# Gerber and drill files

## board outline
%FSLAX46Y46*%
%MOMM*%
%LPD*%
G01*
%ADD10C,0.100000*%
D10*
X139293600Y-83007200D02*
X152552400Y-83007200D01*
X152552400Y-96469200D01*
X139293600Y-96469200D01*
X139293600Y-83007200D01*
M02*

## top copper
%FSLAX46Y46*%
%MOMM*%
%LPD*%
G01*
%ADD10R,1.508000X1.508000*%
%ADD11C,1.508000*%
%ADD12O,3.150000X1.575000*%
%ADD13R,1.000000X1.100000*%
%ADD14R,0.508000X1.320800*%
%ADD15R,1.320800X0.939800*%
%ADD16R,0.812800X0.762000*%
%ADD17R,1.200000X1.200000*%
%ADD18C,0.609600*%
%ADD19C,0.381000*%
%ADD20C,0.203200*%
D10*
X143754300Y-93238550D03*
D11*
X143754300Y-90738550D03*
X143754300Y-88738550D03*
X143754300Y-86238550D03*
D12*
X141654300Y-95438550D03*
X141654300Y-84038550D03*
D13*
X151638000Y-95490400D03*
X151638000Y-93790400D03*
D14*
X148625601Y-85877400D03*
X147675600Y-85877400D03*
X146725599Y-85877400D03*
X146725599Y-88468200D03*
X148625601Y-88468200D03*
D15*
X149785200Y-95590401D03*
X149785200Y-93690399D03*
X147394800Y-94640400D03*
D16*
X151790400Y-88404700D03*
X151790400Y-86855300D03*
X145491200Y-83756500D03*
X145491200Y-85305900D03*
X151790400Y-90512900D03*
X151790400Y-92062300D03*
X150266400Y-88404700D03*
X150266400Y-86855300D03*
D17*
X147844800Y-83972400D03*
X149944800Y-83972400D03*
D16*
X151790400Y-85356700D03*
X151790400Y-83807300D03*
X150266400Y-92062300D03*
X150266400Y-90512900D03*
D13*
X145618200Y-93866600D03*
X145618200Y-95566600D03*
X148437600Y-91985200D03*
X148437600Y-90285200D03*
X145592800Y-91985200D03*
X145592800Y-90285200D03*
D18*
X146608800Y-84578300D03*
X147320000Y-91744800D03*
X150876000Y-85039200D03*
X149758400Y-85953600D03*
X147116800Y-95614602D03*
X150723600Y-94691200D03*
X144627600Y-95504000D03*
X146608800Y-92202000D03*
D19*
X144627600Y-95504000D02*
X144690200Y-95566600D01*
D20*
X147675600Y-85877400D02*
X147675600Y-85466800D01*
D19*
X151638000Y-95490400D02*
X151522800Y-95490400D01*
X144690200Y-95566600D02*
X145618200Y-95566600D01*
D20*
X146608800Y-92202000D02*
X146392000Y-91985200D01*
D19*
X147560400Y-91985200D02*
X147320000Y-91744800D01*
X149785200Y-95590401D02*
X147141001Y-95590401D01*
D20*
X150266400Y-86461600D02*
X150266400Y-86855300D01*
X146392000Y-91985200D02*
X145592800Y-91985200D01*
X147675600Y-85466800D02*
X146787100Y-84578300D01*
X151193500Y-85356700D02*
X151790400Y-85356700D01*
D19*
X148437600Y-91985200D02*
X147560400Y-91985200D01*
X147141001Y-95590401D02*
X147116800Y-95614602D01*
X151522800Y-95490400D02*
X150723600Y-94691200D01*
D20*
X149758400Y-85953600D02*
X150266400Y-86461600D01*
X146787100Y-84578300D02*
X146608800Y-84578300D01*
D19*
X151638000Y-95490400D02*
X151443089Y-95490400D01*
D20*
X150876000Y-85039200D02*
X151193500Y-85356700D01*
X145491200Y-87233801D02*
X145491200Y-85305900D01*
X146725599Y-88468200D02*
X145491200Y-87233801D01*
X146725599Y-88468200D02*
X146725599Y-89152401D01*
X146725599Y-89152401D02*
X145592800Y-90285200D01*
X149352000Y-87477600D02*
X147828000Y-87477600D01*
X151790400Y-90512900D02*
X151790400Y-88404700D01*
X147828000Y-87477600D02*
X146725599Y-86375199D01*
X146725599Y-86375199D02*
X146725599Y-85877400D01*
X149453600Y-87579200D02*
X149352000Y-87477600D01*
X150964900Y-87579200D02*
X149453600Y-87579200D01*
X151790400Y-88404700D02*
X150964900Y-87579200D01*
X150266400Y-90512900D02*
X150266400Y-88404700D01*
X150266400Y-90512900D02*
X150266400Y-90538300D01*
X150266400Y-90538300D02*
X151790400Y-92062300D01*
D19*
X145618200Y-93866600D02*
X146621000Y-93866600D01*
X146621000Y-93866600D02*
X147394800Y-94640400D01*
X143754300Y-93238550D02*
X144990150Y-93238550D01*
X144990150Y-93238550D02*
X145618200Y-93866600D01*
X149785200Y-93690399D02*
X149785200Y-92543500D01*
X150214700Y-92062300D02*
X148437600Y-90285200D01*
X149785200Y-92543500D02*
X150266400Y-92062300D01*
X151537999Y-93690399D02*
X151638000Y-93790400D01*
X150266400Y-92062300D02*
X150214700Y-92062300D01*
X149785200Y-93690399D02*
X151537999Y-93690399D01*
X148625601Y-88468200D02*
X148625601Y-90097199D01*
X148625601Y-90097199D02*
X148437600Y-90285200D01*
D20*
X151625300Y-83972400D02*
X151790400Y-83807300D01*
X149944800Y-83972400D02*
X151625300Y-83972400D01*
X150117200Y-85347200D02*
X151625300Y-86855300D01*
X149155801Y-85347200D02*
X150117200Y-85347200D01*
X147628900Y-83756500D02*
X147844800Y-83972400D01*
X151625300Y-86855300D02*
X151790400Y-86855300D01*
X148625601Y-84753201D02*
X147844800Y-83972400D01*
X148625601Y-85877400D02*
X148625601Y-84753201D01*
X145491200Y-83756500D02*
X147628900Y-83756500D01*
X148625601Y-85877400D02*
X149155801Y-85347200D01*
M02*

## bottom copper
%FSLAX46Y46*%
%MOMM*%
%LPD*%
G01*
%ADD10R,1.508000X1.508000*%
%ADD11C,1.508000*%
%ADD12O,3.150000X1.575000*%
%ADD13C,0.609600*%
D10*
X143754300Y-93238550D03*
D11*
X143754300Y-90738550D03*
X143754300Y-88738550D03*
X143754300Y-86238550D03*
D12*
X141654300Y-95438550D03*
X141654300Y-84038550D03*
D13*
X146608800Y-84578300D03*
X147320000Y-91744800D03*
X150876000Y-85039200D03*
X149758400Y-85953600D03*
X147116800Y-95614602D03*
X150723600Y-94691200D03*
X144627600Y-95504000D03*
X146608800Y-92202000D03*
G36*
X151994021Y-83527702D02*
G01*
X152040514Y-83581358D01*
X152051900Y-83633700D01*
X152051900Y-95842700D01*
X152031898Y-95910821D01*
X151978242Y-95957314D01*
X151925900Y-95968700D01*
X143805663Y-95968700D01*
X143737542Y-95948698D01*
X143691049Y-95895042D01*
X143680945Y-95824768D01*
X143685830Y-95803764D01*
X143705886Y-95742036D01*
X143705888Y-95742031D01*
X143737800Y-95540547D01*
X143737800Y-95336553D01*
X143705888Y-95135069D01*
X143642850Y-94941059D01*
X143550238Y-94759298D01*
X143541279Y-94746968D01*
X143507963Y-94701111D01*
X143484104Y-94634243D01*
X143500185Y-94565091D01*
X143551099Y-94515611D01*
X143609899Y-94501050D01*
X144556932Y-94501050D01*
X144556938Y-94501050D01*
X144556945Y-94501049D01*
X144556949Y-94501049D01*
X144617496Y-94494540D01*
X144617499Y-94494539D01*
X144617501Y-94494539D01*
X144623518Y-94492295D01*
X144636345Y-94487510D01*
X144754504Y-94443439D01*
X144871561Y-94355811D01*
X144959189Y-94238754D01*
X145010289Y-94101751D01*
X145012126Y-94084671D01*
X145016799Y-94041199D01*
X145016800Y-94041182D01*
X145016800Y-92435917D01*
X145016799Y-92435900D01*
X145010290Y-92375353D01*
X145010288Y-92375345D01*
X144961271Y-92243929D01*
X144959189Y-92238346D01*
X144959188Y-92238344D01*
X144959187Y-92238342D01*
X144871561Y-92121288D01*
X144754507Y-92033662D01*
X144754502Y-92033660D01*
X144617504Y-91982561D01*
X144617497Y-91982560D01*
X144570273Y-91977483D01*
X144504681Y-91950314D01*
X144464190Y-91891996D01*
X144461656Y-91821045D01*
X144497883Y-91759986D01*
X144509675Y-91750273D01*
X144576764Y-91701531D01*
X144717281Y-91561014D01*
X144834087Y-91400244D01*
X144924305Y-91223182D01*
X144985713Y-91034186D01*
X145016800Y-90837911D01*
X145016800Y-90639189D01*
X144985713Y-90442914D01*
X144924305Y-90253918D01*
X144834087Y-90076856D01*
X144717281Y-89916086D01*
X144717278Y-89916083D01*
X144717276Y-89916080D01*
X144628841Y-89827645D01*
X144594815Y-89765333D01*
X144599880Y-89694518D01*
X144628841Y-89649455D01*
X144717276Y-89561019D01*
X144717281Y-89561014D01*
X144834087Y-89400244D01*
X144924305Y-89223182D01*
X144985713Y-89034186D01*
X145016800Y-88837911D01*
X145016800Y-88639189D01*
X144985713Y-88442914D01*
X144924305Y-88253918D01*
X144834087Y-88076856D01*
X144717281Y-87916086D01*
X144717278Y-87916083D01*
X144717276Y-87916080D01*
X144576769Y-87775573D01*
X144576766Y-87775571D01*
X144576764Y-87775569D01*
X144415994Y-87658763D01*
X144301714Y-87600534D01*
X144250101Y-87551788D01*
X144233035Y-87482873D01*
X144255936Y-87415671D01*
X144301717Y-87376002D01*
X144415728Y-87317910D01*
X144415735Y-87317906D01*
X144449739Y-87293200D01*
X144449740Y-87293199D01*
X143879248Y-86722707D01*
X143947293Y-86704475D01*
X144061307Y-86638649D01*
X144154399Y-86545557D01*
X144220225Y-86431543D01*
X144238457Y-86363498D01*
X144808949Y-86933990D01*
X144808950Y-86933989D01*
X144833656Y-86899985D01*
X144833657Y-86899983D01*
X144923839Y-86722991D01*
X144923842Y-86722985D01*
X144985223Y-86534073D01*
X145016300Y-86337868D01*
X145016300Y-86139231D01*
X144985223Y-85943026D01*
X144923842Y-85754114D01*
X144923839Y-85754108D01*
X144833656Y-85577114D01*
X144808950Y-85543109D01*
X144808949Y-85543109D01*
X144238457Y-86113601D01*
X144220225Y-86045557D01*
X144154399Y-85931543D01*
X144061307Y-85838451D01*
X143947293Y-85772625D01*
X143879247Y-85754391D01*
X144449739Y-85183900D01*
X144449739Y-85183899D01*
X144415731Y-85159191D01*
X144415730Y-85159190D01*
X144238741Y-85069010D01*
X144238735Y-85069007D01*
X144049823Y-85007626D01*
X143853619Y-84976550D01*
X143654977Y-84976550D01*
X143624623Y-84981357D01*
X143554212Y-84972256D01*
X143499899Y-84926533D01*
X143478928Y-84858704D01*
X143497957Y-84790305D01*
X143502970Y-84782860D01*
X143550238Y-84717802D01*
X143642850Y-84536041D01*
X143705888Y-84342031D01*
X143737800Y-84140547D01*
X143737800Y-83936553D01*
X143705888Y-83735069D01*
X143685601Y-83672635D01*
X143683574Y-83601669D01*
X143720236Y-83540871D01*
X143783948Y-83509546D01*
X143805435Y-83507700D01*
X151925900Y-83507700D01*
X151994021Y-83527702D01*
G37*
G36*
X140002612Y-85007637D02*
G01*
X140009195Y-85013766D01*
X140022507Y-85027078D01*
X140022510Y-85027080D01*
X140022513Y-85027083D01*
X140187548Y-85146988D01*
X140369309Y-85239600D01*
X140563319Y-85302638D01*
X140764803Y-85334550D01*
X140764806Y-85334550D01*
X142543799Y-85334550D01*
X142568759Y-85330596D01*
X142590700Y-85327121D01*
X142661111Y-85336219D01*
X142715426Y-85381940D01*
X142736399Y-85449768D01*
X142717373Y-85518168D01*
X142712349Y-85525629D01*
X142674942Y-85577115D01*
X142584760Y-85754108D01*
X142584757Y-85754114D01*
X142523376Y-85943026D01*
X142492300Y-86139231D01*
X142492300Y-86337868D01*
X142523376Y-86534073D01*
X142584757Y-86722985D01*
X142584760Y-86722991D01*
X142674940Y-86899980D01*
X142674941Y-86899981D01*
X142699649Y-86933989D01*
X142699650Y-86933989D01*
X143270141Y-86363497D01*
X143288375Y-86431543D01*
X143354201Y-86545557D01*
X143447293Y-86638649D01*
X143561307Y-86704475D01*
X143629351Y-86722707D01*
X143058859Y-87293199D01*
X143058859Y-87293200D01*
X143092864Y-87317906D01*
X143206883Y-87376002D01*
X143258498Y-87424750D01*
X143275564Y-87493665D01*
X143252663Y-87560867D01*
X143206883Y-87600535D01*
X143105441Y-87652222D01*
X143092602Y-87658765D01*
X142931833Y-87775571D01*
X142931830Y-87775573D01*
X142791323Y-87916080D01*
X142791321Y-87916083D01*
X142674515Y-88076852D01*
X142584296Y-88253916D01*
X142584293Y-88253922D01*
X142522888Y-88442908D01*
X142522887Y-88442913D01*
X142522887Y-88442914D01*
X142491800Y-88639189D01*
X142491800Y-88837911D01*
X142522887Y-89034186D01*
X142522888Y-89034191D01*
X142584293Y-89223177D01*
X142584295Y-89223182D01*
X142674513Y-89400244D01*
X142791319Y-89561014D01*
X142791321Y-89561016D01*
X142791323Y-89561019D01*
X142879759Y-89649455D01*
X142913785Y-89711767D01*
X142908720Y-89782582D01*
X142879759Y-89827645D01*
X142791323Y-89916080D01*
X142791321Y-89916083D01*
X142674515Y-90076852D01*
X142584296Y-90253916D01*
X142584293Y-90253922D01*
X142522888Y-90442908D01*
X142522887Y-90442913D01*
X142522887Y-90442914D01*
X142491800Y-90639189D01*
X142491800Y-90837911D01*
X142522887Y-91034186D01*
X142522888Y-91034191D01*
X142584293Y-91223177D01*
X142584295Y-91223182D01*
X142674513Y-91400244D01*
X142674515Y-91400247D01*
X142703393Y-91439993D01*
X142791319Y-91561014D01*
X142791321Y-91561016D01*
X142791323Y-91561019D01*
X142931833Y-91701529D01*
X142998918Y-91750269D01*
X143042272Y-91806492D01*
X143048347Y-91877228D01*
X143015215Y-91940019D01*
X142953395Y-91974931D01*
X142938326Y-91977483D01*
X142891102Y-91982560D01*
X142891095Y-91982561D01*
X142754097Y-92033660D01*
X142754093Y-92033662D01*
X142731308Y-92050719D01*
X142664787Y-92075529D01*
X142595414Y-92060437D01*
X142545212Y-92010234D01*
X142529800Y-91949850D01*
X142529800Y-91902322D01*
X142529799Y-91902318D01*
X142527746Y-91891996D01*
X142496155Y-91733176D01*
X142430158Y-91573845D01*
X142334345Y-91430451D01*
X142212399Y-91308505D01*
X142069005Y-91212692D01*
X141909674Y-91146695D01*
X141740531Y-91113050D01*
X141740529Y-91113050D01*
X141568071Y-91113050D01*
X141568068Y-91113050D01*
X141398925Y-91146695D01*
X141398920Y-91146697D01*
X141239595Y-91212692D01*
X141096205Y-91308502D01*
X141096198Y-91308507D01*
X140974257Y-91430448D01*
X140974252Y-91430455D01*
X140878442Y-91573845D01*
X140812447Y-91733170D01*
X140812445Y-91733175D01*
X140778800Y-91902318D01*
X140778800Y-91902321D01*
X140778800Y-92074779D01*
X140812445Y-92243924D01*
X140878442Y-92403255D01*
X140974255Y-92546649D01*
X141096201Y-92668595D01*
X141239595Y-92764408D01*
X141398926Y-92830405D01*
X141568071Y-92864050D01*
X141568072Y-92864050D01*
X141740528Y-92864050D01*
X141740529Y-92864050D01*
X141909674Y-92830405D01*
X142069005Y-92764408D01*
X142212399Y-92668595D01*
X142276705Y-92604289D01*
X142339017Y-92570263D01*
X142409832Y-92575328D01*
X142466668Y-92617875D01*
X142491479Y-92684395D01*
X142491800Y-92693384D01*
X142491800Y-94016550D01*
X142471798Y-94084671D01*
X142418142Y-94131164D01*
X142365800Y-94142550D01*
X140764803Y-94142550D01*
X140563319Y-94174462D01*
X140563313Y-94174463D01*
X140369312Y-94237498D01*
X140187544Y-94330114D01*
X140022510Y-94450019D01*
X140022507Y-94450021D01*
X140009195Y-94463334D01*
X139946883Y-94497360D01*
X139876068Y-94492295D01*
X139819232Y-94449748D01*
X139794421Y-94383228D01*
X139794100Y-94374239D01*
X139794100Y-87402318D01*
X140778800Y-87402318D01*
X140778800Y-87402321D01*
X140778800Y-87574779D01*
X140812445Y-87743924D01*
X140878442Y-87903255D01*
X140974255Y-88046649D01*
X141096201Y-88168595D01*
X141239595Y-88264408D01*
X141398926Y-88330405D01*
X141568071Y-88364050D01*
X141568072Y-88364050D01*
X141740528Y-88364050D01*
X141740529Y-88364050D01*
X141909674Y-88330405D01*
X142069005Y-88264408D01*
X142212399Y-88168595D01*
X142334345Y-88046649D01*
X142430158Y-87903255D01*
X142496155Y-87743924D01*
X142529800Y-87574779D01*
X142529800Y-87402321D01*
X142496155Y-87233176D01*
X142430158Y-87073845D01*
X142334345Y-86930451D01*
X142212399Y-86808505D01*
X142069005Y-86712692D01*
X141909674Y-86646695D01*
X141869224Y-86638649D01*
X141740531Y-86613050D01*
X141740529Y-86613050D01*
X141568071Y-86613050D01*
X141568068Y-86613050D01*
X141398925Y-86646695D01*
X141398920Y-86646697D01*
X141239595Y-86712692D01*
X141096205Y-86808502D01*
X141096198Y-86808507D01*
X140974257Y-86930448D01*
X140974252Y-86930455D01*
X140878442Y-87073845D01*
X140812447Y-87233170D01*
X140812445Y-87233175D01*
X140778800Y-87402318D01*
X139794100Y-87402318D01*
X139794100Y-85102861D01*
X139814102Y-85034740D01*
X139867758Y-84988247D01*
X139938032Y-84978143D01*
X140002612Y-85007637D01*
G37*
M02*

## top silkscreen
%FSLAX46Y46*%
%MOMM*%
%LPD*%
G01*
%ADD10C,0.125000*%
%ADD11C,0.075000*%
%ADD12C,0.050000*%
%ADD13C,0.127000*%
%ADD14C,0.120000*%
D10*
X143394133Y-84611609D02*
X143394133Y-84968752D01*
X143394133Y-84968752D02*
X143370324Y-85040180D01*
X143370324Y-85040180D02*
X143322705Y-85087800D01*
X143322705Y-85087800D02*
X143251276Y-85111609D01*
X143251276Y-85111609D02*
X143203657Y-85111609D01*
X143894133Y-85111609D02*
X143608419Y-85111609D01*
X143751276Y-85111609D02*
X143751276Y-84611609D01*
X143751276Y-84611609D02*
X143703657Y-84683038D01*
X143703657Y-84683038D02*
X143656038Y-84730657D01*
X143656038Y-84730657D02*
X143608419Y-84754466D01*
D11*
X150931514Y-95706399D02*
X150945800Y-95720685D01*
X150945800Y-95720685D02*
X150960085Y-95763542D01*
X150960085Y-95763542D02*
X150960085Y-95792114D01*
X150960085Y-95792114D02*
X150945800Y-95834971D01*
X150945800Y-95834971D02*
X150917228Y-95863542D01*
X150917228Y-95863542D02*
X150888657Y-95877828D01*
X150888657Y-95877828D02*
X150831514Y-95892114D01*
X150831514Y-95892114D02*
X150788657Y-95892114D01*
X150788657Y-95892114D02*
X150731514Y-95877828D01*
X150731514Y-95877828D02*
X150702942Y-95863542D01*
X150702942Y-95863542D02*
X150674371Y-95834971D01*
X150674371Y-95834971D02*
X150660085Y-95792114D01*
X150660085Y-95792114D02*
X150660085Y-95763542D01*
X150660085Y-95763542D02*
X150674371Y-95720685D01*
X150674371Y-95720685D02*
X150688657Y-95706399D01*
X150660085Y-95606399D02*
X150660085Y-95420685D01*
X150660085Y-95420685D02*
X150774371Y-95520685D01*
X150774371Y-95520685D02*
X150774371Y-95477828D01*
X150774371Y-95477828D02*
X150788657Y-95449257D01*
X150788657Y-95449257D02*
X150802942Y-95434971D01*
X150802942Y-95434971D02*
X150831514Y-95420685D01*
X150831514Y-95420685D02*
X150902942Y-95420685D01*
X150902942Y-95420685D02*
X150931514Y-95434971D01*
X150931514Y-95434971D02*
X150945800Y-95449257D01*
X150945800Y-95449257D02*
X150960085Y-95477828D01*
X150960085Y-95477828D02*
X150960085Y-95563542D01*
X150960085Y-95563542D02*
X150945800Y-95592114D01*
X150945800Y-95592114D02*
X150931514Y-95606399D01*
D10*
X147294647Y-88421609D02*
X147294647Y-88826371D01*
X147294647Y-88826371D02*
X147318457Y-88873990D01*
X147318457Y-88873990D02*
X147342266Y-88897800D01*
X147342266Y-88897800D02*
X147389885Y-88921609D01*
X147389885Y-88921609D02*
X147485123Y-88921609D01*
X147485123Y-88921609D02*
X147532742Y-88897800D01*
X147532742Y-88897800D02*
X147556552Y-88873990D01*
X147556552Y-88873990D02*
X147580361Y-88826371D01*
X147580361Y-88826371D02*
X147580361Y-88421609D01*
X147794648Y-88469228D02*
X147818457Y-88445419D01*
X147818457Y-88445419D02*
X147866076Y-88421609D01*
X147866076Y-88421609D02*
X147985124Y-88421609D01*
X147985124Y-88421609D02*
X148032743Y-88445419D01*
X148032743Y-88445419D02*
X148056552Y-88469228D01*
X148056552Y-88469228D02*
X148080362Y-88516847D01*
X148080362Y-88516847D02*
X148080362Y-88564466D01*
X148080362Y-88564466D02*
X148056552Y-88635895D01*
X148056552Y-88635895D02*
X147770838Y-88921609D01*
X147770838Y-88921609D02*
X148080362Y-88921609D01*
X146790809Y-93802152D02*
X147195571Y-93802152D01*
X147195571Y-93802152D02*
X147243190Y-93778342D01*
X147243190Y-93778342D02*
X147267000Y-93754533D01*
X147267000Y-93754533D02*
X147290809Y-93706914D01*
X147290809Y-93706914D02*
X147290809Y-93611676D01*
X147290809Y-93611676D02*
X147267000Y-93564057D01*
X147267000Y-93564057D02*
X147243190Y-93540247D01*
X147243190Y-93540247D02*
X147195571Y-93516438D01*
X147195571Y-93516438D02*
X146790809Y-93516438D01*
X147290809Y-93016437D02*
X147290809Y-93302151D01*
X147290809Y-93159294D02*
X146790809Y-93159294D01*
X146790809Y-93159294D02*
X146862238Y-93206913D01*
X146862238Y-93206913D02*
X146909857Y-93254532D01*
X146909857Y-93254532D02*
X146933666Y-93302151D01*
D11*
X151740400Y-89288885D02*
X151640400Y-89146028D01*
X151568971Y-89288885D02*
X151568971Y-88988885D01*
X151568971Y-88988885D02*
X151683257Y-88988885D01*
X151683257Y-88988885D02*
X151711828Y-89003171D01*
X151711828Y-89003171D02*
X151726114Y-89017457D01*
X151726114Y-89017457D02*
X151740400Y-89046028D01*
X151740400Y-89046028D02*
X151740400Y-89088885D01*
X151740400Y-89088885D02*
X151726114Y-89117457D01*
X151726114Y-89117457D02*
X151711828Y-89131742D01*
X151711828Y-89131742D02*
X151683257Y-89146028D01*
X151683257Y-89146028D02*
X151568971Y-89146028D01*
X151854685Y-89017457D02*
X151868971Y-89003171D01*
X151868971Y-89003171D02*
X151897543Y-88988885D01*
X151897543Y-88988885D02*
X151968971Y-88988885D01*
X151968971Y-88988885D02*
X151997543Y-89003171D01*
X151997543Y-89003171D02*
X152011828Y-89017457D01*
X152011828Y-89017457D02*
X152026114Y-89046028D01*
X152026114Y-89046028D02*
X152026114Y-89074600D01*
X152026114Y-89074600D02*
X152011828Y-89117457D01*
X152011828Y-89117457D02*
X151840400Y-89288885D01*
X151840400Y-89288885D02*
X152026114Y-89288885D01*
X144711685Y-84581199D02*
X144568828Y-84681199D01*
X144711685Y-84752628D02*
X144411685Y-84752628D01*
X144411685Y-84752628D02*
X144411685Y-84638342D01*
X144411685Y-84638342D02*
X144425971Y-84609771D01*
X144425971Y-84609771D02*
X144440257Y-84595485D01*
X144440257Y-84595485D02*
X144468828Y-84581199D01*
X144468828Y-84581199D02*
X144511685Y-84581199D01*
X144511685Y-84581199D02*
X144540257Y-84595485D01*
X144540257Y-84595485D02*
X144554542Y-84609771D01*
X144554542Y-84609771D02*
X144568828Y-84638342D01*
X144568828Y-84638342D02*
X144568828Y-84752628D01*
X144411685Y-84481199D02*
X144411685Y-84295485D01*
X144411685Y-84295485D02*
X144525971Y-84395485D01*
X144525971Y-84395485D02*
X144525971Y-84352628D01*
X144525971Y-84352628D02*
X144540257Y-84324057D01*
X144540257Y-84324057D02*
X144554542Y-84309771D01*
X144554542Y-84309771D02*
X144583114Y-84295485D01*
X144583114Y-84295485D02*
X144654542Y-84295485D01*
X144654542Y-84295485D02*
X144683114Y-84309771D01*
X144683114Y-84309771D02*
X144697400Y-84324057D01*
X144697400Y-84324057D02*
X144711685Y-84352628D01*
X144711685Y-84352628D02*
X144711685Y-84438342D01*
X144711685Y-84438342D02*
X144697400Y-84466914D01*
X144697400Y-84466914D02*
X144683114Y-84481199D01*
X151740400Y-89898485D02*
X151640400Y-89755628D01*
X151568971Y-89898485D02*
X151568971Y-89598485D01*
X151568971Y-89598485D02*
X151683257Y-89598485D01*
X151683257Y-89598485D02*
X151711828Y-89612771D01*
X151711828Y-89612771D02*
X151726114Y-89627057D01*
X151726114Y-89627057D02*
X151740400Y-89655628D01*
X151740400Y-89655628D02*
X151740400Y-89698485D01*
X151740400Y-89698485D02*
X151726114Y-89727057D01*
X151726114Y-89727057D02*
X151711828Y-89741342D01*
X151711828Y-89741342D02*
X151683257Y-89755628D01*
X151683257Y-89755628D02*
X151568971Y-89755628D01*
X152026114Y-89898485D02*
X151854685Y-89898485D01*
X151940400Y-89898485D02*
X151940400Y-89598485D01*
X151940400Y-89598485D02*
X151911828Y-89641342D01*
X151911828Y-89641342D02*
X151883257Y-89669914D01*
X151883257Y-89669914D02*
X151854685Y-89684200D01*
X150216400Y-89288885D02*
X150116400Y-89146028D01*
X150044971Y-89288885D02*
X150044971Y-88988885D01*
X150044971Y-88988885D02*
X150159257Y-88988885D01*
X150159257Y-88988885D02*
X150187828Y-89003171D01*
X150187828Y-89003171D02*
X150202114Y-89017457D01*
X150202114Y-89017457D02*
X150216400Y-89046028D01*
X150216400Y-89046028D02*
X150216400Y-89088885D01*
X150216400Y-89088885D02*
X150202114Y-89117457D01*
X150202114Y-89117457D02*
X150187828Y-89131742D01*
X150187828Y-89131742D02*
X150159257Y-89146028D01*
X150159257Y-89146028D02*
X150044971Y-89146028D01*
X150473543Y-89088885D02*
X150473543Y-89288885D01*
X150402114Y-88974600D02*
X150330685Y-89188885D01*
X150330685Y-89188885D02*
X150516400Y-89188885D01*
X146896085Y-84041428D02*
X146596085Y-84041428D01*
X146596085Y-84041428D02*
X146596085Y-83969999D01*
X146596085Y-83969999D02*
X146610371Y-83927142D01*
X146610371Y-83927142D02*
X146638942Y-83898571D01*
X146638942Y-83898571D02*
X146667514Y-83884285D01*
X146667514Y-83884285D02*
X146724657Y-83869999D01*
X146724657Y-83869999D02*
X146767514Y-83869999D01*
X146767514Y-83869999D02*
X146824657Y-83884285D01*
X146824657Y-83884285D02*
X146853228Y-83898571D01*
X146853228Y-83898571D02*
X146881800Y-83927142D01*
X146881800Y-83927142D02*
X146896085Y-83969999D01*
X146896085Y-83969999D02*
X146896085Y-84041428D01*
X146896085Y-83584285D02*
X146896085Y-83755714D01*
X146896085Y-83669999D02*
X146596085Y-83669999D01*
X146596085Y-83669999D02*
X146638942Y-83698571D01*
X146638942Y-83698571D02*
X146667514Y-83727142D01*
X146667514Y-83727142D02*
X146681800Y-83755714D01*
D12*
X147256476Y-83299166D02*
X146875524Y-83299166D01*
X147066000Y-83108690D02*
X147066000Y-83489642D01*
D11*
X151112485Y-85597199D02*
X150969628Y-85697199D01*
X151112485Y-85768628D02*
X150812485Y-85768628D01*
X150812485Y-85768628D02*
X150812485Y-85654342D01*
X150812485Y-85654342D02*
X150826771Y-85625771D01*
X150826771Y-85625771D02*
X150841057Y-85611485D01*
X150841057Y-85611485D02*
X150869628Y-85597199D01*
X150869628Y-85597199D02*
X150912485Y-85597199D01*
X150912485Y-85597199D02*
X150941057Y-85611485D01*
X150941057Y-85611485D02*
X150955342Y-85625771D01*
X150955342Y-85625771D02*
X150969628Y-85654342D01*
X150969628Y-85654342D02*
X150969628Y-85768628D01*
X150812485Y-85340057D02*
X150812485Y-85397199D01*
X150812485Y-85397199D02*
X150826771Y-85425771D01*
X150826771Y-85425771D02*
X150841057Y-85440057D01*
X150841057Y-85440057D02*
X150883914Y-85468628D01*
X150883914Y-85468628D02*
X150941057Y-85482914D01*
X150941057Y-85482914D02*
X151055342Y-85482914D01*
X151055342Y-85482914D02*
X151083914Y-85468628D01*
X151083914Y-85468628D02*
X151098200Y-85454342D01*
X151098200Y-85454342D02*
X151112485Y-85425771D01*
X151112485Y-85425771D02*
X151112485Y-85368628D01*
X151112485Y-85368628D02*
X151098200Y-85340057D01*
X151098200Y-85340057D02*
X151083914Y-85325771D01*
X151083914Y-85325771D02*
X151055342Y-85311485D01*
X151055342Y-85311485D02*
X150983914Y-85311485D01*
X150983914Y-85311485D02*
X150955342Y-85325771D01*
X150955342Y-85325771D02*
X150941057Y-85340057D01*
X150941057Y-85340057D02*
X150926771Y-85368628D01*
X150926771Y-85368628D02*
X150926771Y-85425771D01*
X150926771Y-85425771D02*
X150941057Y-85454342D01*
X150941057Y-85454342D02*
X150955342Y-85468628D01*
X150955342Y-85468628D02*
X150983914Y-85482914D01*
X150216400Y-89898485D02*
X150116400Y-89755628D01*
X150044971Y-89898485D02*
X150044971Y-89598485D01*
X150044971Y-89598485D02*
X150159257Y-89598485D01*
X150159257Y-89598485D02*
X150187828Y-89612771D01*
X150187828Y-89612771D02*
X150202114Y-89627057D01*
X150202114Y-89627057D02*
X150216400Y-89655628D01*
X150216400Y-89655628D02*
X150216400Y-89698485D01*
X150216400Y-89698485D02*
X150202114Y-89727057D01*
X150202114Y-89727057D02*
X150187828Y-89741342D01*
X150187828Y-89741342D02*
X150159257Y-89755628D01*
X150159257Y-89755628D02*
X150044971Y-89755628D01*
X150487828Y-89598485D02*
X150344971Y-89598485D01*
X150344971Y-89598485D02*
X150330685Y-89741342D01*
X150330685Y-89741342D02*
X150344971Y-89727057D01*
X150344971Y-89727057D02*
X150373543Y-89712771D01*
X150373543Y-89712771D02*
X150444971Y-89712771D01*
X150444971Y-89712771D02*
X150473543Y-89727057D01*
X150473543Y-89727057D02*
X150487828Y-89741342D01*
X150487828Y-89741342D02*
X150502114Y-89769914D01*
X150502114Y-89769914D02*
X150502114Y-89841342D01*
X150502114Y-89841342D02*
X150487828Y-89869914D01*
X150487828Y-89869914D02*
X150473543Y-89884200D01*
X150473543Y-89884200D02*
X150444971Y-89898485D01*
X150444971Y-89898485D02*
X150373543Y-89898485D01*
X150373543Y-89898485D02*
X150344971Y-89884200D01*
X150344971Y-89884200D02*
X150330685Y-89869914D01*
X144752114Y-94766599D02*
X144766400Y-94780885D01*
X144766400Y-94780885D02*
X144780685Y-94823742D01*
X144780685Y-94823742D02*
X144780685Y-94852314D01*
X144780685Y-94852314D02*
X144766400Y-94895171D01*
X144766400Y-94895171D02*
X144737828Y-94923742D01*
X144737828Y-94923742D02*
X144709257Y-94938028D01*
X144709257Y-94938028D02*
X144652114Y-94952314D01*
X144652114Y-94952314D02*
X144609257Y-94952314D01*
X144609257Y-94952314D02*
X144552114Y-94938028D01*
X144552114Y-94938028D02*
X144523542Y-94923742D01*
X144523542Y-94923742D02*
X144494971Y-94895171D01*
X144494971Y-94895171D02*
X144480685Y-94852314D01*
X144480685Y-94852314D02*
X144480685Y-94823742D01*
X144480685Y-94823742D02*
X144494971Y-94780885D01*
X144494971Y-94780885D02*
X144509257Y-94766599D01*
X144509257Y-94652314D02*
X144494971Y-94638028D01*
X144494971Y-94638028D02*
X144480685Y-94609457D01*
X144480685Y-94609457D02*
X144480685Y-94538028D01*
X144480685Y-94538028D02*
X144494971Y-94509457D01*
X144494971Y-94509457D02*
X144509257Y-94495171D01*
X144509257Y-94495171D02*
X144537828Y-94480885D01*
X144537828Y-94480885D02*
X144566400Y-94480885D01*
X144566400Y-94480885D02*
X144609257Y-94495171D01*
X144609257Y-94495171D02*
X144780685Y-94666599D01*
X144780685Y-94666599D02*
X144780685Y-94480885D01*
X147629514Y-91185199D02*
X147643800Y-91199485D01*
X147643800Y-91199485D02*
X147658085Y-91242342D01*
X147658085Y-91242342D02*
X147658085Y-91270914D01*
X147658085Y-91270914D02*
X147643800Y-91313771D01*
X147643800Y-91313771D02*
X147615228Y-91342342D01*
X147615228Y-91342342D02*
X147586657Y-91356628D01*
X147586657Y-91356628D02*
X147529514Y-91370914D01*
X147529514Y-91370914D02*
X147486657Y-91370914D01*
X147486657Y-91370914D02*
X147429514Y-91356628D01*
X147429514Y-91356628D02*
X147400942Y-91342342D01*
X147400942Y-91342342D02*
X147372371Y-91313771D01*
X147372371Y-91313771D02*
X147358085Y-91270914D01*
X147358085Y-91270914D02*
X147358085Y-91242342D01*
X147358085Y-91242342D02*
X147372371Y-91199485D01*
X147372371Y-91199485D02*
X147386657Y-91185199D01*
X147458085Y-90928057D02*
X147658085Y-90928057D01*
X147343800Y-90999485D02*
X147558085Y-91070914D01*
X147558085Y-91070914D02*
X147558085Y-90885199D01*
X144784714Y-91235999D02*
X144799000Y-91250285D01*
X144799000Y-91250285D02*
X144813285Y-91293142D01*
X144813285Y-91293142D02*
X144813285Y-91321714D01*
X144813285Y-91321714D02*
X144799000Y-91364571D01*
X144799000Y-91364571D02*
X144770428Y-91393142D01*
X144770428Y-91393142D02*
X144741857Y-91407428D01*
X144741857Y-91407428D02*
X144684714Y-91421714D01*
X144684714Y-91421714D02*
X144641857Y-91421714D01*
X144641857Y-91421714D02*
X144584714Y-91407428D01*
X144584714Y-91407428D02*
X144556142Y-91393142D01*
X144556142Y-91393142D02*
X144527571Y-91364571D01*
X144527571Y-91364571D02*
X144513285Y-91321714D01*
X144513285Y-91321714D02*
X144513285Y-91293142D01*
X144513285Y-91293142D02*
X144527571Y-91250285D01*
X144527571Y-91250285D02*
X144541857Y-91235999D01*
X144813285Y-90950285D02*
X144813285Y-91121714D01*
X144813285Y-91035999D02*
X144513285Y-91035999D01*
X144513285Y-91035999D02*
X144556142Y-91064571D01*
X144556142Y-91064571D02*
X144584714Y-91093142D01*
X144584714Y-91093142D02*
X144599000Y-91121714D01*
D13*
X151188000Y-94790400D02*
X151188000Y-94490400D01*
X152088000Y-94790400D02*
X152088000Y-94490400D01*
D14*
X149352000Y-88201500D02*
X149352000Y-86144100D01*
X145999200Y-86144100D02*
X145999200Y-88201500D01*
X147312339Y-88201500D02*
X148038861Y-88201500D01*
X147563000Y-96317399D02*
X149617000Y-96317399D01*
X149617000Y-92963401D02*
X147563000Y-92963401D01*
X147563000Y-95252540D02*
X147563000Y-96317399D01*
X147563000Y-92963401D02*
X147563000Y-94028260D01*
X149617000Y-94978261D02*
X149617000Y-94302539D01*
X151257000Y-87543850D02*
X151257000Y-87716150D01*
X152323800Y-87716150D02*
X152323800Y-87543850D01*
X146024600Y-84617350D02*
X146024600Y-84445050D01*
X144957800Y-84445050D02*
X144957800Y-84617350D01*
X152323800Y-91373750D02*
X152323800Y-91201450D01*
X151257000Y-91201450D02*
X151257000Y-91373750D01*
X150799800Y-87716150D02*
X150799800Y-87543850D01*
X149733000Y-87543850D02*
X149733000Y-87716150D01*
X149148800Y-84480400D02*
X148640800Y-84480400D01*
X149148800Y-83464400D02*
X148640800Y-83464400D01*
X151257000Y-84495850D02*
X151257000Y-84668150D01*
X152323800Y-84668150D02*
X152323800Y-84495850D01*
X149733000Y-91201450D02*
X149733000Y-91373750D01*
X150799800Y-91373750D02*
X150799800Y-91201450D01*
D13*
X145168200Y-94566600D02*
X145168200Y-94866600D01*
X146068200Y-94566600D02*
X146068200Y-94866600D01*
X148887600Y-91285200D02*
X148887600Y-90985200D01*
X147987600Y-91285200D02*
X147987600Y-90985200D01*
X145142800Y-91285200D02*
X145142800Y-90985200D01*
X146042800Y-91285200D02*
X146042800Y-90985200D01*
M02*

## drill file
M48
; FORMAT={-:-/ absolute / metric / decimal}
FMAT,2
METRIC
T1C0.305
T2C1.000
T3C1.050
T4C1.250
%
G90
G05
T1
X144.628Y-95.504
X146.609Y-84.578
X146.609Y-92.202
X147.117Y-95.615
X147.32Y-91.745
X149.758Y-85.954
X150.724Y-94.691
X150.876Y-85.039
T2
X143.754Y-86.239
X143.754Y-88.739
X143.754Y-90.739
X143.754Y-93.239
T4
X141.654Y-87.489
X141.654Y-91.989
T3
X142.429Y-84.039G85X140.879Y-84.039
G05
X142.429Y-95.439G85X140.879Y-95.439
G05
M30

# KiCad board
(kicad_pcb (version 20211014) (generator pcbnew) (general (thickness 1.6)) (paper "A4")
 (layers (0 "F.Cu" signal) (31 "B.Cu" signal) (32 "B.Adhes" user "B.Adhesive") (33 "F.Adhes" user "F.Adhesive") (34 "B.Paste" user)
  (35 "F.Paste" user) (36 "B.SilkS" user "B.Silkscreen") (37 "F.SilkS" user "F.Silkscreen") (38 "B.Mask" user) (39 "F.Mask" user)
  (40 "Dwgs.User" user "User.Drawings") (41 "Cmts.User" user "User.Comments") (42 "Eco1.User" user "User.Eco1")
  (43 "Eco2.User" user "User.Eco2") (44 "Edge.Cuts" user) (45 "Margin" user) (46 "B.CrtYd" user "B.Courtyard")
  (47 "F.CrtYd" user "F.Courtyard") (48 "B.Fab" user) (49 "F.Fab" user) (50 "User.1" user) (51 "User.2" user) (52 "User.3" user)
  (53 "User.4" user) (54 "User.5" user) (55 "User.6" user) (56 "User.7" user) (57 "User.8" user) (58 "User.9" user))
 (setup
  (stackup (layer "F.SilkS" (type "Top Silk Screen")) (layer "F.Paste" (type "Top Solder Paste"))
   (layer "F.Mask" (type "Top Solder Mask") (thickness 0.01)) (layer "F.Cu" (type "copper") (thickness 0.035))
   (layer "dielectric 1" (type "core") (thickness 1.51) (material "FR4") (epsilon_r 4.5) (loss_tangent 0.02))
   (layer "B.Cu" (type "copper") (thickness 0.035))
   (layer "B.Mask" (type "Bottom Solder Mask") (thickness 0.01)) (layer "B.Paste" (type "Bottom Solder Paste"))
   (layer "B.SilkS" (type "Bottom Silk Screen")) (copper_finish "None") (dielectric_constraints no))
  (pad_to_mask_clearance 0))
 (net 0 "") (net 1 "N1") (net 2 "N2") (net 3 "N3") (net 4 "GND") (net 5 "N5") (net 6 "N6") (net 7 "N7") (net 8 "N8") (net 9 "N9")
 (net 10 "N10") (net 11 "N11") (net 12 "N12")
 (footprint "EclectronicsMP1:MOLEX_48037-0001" (layer "F.Cu") (at 141.6543 89.73855 -90)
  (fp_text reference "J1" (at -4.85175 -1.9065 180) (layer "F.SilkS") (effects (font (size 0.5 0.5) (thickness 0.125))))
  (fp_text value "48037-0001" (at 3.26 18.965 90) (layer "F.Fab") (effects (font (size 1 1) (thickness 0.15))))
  (pad "" np_thru_hole circle (at -2.25 0 270) (size 1.25 1.25) (drill 1.25) (layers *.Cu *.Mask))
  (pad "" np_thru_hole circle (at 2.25 0 270) (size 1.25 1.25) (drill 1.25) (layers *.Cu *.Mask))
  (pad "1" thru_hole rect (at 3.5 -2.1 270) (size 1.508 1.508) (drill 1) (layers *.Cu *.Mask) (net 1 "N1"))
  (pad "2" thru_hole circle (at 1 -2.1 270) (size 1.508 1.508) (drill 1) (layers *.Cu *.Mask) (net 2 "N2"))
  (pad "3" thru_hole circle (at -1 -2.1 270) (size 1.508 1.508) (drill 1) (layers *.Cu *.Mask) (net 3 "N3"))
  (pad "4" thru_hole circle (at -3.5 -2.1 270) (size 1.508 1.508) (drill 1) (layers *.Cu *.Mask) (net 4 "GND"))
  (pad "S1" thru_hole oval (at 5.7 0 270) (size 1.575 3.15) (drill oval 1.05 2.6) (layers *.Cu *.Mask) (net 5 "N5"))
  (pad "S2" thru_hole oval (at -5.7 0 270) (size 1.575 3.15) (drill oval 1.05 2.6) (layers *.Cu *.Mask) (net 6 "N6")))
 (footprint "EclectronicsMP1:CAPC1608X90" (layer "F.Cu") (at 151.638 94.6404 90)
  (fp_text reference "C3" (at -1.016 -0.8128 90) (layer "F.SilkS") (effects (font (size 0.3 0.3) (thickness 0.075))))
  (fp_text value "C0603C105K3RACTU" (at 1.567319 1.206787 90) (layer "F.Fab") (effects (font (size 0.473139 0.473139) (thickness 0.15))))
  (fp_line (start -0.15 -0.45) (end 0.15 -0.45) (layer "F.SilkS") (width 0.127))
  (fp_line (start -0.15 0.45) (end 0.15 0.45) (layer "F.SilkS") (width 0.127))
  (pad "1" smd rect (at -0.85 0 90) (size 1.1 1) (layers "F.Cu" "F.Paste" "F.Mask") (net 4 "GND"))
  (pad "2" smd rect (at 0.85 0 90) (size 1.1 1) (layers "F.Cu" "F.Paste" "F.Mask") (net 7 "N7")))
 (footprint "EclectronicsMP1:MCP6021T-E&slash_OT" (layer "F.Cu") (at 147.6756 87.1728 -90)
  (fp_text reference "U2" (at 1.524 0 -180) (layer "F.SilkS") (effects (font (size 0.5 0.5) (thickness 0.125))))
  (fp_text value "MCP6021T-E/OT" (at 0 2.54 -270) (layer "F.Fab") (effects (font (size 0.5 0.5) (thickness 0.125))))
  (fp_line (start 1.0287 -1.6764) (end -1.0287 -1.6764) (layer "F.SilkS") (width 0.12))
  (fp_line (start -1.0287 1.6764) (end 1.0287 1.6764) (layer "F.SilkS") (width 0.12))
  (fp_line (start 1.0287 0.363261) (end 1.0287 -0.363261) (layer "F.SilkS") (width 0.12))
  (pad "1" smd rect (at -1.2954 -0.950001 270) (size 1.3208 0.508) (layers "F.Cu" "F.Paste" "F.Mask") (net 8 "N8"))
  (pad "2" smd rect (at -1.2954 0 270) (size 1.3208 0.508) (layers "F.Cu" "F.Paste" "F.Mask") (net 4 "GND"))
  (pad "3" smd rect (at -1.2954 0.950001 270) (size 1.3208 0.508) (layers "F.Cu" "F.Paste" "F.Mask") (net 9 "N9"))
  (pad "4" smd rect (at 1.2954 0.950001 270) (size 1.3208 0.508) (layers "F.Cu" "F.Paste" "F.Mask") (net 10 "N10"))
  (pad "5" smd rect (at 1.2954 -0.950001 270) (size 1.3208 0.508) (layers "F.Cu" "F.Paste" "F.Mask") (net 7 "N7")))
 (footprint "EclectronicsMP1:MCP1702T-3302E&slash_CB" (layer "F.Cu") (at 148.59 94.6404 90)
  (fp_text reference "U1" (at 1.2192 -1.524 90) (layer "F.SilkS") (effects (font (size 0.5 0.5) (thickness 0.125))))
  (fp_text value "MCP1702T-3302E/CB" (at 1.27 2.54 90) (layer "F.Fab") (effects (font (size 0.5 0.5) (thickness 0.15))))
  (fp_line (start -1.676999 -1.027) (end -1.676999 1.027) (layer "F.SilkS") (width 0.12))
  (fp_line (start 1.676999 1.027) (end 1.676999 -1.027) (layer "F.SilkS") (width 0.12))
  (fp_line (start -0.61214 -1.027) (end -1.676999 -1.027) (layer "F.SilkS") (width 0.12))
  (fp_line (start 1.676999 -1.027) (end 0.61214 -1.027) (layer "F.SilkS") (width 0.12))
  (fp_line (start -0.337861 1.027) (end 0.337861 1.027) (layer "F.SilkS") (width 0.12))
  (pad "1" smd rect (at -0.950001 1.1952 90) (size 0.9398 1.3208) (layers "F.Cu" "F.Paste" "F.Mask") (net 4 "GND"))
  (pad "2" smd rect (at 0.950001 1.1952 90) (size 0.9398 1.3208) (layers "F.Cu" "F.Paste" "F.Mask") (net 7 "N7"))
  (pad "3" smd rect (at 0 -1.1952 90) (size 0.9398 1.3208) (layers "F.Cu" "F.Paste" "F.Mask") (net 1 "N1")))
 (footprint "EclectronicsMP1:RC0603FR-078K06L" (layer "F.Cu") (at 151.7904 87.63 90)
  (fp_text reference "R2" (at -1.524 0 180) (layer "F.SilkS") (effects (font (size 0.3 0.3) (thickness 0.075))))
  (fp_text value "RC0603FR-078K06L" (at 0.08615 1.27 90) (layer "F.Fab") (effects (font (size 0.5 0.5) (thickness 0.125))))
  (fp_line (start 0.08615 -0.5334) (end -0.08615 -0.5334) (layer "F.SilkS") (width 0.12))
  (fp_line (start -0.08615 0.5334) (end 0.08615 0.5334) (layer "F.SilkS") (width 0.12))
  (pad "1" smd rect (at -0.7747 0 90) (size 0.762 0.8128) (layers "F.Cu" "F.Paste" "F.Mask") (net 9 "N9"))
  (pad "2" smd rect (at 0.7747 0 90) (size 0.762 0.8128) (layers "F.Cu" "F.Paste" "F.Mask") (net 8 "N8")))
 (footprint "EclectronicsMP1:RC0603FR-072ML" (layer "F.Cu") (at 145.4912 84.5312 -90)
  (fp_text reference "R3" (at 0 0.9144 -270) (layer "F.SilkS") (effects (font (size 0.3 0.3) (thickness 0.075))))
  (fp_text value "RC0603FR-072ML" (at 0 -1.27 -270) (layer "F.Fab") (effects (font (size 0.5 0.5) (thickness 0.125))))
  (fp_line (start 0.08615 -0.5334) (end -0.08615 -0.5334) (layer "F.SilkS") (width 0.12))
  (fp_line (start -0.08615 0.5334) (end 0.08615 0.5334) (layer "F.SilkS") (width 0.12))
  (pad "1" smd rect (at -0.7747 0 270) (size 0.762 0.8128) (layers "F.Cu" "F.Paste" "F.Mask") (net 8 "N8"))
  (pad "2" smd rect (at 0.7747 0 270) (size 0.762 0.8128) (layers "F.Cu" "F.Paste" "F.Mask") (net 10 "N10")))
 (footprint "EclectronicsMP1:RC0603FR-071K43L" (layer "F.Cu") (at 151.7904 91.2876 -90)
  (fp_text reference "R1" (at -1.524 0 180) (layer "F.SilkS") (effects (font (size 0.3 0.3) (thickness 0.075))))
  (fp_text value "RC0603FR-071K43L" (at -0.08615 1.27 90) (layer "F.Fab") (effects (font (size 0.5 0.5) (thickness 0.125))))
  (fp_line (start 0.08615 -0.5334) (end -0.08615 -0.5334) (layer "F.SilkS") (width 0.12))
  (fp_line (start -0.08615 0.5334) (end 0.08615 0.5334) (layer "F.SilkS") (width 0.12))
  (pad "1" smd rect (at -0.7747 0 270) (size 0.762 0.8128) (layers "F.Cu" "F.Paste" "F.Mask") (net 9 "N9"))
  (pad "2" smd rect (at 0.7747 0 270) (size 0.762 0.8128) (layers "F.Cu" "F.Paste" "F.Mask") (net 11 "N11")))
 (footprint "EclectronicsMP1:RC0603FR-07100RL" (layer "F.Cu") (at 150.2664 87.63 90)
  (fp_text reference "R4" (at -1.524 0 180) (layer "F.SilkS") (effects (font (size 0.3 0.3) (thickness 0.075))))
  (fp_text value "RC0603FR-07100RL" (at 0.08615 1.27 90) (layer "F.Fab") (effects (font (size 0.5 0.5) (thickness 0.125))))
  (fp_line (start -0.08615 0.5334) (end 0.08615 0.5334) (layer "F.SilkS") (width 0.12))
  (fp_line (start 0.08615 -0.5334) (end -0.08615 -0.5334) (layer "F.SilkS") (width 0.12))
  (pad "1" smd rect (at -0.7747 0 90) (size 0.762 0.8128) (layers "F.Cu" "F.Paste" "F.Mask") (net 11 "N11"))
  (pad "2" smd rect (at 0.7747 0 90) (size 0.762 0.8128) (layers "F.Cu" "F.Paste" "F.Mask") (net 4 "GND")))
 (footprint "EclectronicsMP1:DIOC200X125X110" (layer "F.Cu") (at 148.8948 83.9724 180)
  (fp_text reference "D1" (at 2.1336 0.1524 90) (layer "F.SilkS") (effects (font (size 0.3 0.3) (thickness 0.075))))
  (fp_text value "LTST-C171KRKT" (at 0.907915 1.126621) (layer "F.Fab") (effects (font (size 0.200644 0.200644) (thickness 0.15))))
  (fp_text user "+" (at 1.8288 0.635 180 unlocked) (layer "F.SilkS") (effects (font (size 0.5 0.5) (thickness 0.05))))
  (fp_line (start -0.254 -0.508) (end 0.254 -0.508) (layer "F.SilkS") (width 0.12))
  (fp_line (start -0.254 0.508) (end 0.254 0.508) (layer "F.SilkS") (width 0.12))
  (pad "+" smd rect (at 1.05 0 180) (size 1.2 1.2) (layers "F.Cu" "F.Paste" "F.Mask") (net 8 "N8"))
  (pad "-" smd rect (at -1.05 0 180) (size 1.2 1.2) (layers "F.Cu" "F.Paste" "F.Mask") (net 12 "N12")))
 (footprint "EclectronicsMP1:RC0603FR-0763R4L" (layer "F.Cu") (at 151.7904 84.582 90)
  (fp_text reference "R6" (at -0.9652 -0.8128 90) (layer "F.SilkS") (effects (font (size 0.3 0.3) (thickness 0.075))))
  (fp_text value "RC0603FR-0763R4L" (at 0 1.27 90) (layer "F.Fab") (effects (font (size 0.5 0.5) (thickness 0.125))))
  (fp_line (start 0.08615 -0.5334) (end -0.08615 -0.5334) (layer "F.SilkS") (width 0.12))
  (fp_line (start -0.08615 0.5334) (end 0.08615 0.5334) (layer "F.SilkS") (width 0.12))
  (pad "1" smd rect (at -0.7747 0 90) (size 0.762 0.8128) (layers "F.Cu" "F.Paste" "F.Mask") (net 4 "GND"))
  (pad "2" smd rect (at 0.7747 0 90) (size 0.762 0.8128) (layers "F.Cu" "F.Paste" "F.Mask") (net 12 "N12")))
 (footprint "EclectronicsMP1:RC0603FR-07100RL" (layer "F.Cu") (at 150.2664 91.2876 90)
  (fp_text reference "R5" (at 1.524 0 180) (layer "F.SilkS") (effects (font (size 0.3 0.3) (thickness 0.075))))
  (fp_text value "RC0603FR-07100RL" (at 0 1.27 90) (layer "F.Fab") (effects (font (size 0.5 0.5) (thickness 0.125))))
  (fp_line (start 0.08615 -0.5334) (end -0.08615 -0.5334) (layer "F.SilkS") (width 0.12))
  (fp_line (start -0.08615 0.5334) (end 0.08615 0.5334) (layer "F.SilkS") (width 0.12))
  (pad "1" smd rect (at -0.7747 0 90) (size 0.762 0.8128) (layers "F.Cu" "F.Paste" "F.Mask") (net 7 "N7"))
  (pad "2" smd rect (at 0.7747 0 90) (size 0.762 0.8128) (layers "F.Cu" "F.Paste" "F.Mask") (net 11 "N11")))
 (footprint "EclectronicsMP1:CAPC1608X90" (layer "F.Cu") (at 145.6182 94.7166 -90)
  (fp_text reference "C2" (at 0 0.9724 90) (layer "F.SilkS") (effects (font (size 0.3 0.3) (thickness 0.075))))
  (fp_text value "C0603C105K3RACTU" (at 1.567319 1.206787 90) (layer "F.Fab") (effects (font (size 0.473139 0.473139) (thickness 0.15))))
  (fp_line (start -0.15 0.45) (end 0.15 0.45) (layer "F.SilkS") (width 0.127))
  (fp_line (start -0.15 -0.45) (end 0.15 -0.45) (layer "F.SilkS") (width 0.127))
  (pad "1" smd rect (at -0.85 0 270) (size 1.1 1) (layers "F.Cu" "F.Paste" "F.Mask") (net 1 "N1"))
  (pad "2" smd rect (at 0.85 0 270) (size 1.1 1) (layers "F.Cu" "F.Paste" "F.Mask") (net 4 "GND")))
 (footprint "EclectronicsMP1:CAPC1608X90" (layer "F.Cu") (at 148.4376 91.1352 90)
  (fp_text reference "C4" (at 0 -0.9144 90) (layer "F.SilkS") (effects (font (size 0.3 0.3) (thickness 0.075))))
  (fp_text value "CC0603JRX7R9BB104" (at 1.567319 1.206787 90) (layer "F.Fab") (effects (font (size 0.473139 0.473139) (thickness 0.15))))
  (fp_line (start -0.15 0.45) (end 0.15 0.45) (layer "F.SilkS") (width 0.127))
  (fp_line (start -0.15 -0.45) (end 0.15 -0.45) (layer "F.SilkS") (width 0.127))
  (pad "1" smd rect (at -0.85 0 90) (size 1.1 1) (layers "F.Cu" "F.Paste" "F.Mask") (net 4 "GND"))
  (pad "2" smd rect (at 0.85 0 90) (size 1.1 1) (layers "F.Cu" "F.Paste" "F.Mask") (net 7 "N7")))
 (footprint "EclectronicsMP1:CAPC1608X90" (layer "F.Cu") (at 145.5928 91.1352 90)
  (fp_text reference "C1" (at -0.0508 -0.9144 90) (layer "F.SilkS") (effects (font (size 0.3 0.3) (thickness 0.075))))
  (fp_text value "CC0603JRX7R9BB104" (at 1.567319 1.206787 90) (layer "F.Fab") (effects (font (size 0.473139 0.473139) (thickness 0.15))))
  (fp_line (start -0.15 -0.45) (end 0.15 -0.45) (layer "F.SilkS") (width 0.127))
  (fp_line (start -0.15 0.45) (end 0.15 0.45) (layer "F.SilkS") (width 0.127))
  (pad "1" smd rect (at -0.85 0 90) (size 1.1 1) (layers "F.Cu" "F.Paste" "F.Mask") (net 4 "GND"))
  (pad "2" smd rect (at 0.85 0 90) (size 1.1 1) (layers "F.Cu" "F.Paste" "F.Mask") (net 10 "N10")))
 (gr_rect (start 152.5524 96.4692) (end 139.2936 83.0072) (layer "Edge.Cuts") (width 0.1) (fill none))
 (segment (start 144.6276 95.504) (end 144.6902 95.5666) (width 0.381) (layer "F.Cu") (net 4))
 (segment (start 147.6756 85.8774) (end 147.6756 85.4668) (width 0.2032) (layer "F.Cu") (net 4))
 (segment (start 151.638 95.4904) (end 151.5228 95.4904) (width 0.381) (layer "F.Cu") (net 4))
 (segment (start 144.6902 95.5666) (end 145.6182 95.5666) (width 0.381) (layer "F.Cu") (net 4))
 (segment (start 146.6088 92.202) (end 146.392 91.9852) (width 0.2032) (layer "F.Cu") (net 4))
 (segment (start 147.5604 91.9852) (end 147.32 91.7448) (width 0.381) (layer "F.Cu") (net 4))
 (segment (start 149.7852 95.590401) (end 147.141001 95.590401) (width 0.381) (layer "F.Cu") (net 4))
 (segment (start 150.2664 86.4616) (end 150.2664 86.8553) (width 0.2032) (layer "F.Cu") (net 4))
 (segment (start 146.392 91.9852) (end 145.5928 91.9852) (width 0.2032) (layer "F.Cu") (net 4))
 (segment (start 147.6756 85.4668) (end 146.7871 84.5783) (width 0.2032) (layer "F.Cu") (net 4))
 (segment (start 151.1935 85.3567) (end 151.7904 85.3567) (width 0.2032) (layer "F.Cu") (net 4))
 (segment (start 148.4376 91.9852) (end 147.5604 91.9852) (width 0.381) (layer "F.Cu") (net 4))
 (segment (start 147.141001 95.590401) (end 147.1168 95.614602) (width 0.381) (layer "F.Cu") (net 4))
 (segment (start 151.5228 95.4904) (end 150.7236 94.6912) (width 0.381) (layer "F.Cu") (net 4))
 (segment (start 149.7584 85.9536) (end 150.2664 86.4616) (width 0.2032) (layer "F.Cu") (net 4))
 (segment (start 146.7871 84.5783) (end 146.6088 84.5783) (width 0.2032) (layer "F.Cu") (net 4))
 (segment (start 151.638 95.4904) (end 151.443089 95.4904) (width 0.381) (layer "F.Cu") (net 4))
 (segment (start 150.876 85.0392) (end 151.1935 85.3567) (width 0.2032) (layer "F.Cu") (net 4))
 (via (at 146.6088 84.5783) (size 0.6096) (drill 0.3048) (layers "F.Cu" "B.Cu") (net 4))
 (via (at 147.32 91.7448) (size 0.6096) (drill 0.3048) (layers "F.Cu" "B.Cu") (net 4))
 (via (at 150.876 85.0392) (size 0.6096) (drill 0.3048) (layers "F.Cu" "B.Cu") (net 4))
 (via (at 149.7584 85.9536) (size 0.6096) (drill 0.3048) (layers "F.Cu" "B.Cu") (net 4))
 (via (at 147.1168 95.614602) (size 0.6096) (drill 0.3048) (layers "F.Cu" "B.Cu") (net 4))
 (via (at 150.7236 94.6912) (size 0.6096) (drill 0.3048) (layers "F.Cu" "B.Cu") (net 4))
 (via (at 144.6276 95.504) (size 0.6096) (drill 0.3048) (layers "F.Cu" "B.Cu") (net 4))
 (via (at 146.6088 92.202) (size 0.6096) (drill 0.3048) (layers "F.Cu" "B.Cu") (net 4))
 (segment (start 145.4912 87.233801) (end 145.4912 85.3059) (width 0.2032) (layer "F.Cu") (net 10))
 (segment (start 146.725599 88.4682) (end 145.4912 87.233801) (width 0.2032) (layer "F.Cu") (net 10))
 (segment (start 146.725599 88.4682) (end 146.725599 89.152401) (width 0.2032) (layer "F.Cu") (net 10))
 (segment (start 146.725599 89.152401) (end 145.5928 90.2852) (width 0.2032) (layer "F.Cu") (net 10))
 (segment (start 149.352 87.4776) (end 147.828 87.4776) (width 0.2032) (layer "F.Cu") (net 9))
 (segment (start 151.7904 90.5129) (end 151.7904 88.4047) (width 0.2032) (layer "F.Cu") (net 9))
 (segment (start 147.828 87.4776) (end 146.725599 86.375199) (width 0.2032) (layer "F.Cu") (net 9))
 (segment (start 146.725599 86.375199) (end 146.725599 85.8774) (width 0.2032) (layer "F.Cu") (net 9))
 (segment (start 149.4536 87.5792) (end 149.352 87.4776) (width 0.2032) (layer "F.Cu") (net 9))
 (segment (start 150.9649 87.5792) (end 149.4536 87.5792) (width 0.2032) (layer "F.Cu") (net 9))
 (segment (start 151.7904 88.4047) (end 150.9649 87.5792) (width 0.2032) (layer "F.Cu") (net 9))
 (segment (start 150.2664 90.5129) (end 150.2664 88.4047) (width 0.2032) (layer "F.Cu") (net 11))
 (segment (start 150.2664 90.5129) (end 150.2664 90.5383) (width 0.2032) (layer "F.Cu") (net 11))
 (segment (start 150.2664 90.5383) (end 151.7904 92.0623) (width 0.2032) (layer "F.Cu") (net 11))
 (segment (start 145.6182 93.8666) (end 146.621 93.8666) (width 0.381) (layer "F.Cu") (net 1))
 (segment (start 146.621 93.8666) (end 147.3948 94.6404) (width 0.381) (layer "F.Cu") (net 1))
 (segment (start 143.7543 93.23855) (end 144.99015 93.23855) (width 0.381) (layer "F.Cu") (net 1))
 (segment (start 144.99015 93.23855) (end 145.6182 93.8666) (width 0.381) (layer "F.Cu") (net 1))
 (segment (start 149.7852 93.690399) (end 149.7852 92.5435) (width 0.381) (layer "F.Cu") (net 7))
 (segment (start 150.2147 92.0623) (end 148.4376 90.2852) (width 0.381) (layer "F.Cu") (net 7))
 (segment (start 149.7852 92.5435) (end 150.2664 92.0623) (width 0.381) (layer "F.Cu") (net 7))
 (segment (start 151.537999 93.690399) (end 151.638 93.7904) (width 0.381) (layer "F.Cu") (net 7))
 (segment (start 150.2664 92.0623) (end 150.2147 92.0623) (width 0.381) (layer "F.Cu") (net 7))
 (segment (start 149.7852 93.690399) (end 151.537999 93.690399) (width 0.381) (layer "F.Cu") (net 7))
 (segment (start 148.625601 88.4682) (end 148.625601 90.097199) (width 0.381) (layer "F.Cu") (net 7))
 (segment (start 148.625601 90.097199) (end 148.4376 90.2852) (width 0.381) (layer "F.Cu") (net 7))
 (segment (start 151.6253 83.9724) (end 151.7904 83.8073) (width 0.2032) (layer "F.Cu") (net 12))
 (segment (start 149.9448 83.9724) (end 151.6253 83.9724) (width 0.2032) (layer "F.Cu") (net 12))
 (segment (start 150.1172 85.3472) (end 151.6253 86.8553) (width 0.2032) (layer "F.Cu") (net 8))
 (segment (start 149.155801 85.3472) (end 150.1172 85.3472) (width 0.2032) (layer "F.Cu") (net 8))
 (segment (start 147.6289 83.7565) (end 147.8448 83.9724) (width 0.2032) (layer "F.Cu") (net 8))
 (segment (start 151.6253 86.8553) (end 151.7904 86.8553) (width 0.2032) (layer "F.Cu") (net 8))
 (segment (start 148.625601 84.753201) (end 147.8448 83.9724) (width 0.2032) (layer "F.Cu") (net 8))
 (segment (start 148.625601 85.8774) (end 148.625601 84.753201) (width 0.2032) (layer "F.Cu") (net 8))
 (segment (start 145.4912 83.7565) (end 147.6289 83.7565) (width 0.2032) (layer "F.Cu") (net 8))
 (segment (start 148.625601 85.8774) (end 149.155801 85.3472) (width 0.2032) (layer "F.Cu") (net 8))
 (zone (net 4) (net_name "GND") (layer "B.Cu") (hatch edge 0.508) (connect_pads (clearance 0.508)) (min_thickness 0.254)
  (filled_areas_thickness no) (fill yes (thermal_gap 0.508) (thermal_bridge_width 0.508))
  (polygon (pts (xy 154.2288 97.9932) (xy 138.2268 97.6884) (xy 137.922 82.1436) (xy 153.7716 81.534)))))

